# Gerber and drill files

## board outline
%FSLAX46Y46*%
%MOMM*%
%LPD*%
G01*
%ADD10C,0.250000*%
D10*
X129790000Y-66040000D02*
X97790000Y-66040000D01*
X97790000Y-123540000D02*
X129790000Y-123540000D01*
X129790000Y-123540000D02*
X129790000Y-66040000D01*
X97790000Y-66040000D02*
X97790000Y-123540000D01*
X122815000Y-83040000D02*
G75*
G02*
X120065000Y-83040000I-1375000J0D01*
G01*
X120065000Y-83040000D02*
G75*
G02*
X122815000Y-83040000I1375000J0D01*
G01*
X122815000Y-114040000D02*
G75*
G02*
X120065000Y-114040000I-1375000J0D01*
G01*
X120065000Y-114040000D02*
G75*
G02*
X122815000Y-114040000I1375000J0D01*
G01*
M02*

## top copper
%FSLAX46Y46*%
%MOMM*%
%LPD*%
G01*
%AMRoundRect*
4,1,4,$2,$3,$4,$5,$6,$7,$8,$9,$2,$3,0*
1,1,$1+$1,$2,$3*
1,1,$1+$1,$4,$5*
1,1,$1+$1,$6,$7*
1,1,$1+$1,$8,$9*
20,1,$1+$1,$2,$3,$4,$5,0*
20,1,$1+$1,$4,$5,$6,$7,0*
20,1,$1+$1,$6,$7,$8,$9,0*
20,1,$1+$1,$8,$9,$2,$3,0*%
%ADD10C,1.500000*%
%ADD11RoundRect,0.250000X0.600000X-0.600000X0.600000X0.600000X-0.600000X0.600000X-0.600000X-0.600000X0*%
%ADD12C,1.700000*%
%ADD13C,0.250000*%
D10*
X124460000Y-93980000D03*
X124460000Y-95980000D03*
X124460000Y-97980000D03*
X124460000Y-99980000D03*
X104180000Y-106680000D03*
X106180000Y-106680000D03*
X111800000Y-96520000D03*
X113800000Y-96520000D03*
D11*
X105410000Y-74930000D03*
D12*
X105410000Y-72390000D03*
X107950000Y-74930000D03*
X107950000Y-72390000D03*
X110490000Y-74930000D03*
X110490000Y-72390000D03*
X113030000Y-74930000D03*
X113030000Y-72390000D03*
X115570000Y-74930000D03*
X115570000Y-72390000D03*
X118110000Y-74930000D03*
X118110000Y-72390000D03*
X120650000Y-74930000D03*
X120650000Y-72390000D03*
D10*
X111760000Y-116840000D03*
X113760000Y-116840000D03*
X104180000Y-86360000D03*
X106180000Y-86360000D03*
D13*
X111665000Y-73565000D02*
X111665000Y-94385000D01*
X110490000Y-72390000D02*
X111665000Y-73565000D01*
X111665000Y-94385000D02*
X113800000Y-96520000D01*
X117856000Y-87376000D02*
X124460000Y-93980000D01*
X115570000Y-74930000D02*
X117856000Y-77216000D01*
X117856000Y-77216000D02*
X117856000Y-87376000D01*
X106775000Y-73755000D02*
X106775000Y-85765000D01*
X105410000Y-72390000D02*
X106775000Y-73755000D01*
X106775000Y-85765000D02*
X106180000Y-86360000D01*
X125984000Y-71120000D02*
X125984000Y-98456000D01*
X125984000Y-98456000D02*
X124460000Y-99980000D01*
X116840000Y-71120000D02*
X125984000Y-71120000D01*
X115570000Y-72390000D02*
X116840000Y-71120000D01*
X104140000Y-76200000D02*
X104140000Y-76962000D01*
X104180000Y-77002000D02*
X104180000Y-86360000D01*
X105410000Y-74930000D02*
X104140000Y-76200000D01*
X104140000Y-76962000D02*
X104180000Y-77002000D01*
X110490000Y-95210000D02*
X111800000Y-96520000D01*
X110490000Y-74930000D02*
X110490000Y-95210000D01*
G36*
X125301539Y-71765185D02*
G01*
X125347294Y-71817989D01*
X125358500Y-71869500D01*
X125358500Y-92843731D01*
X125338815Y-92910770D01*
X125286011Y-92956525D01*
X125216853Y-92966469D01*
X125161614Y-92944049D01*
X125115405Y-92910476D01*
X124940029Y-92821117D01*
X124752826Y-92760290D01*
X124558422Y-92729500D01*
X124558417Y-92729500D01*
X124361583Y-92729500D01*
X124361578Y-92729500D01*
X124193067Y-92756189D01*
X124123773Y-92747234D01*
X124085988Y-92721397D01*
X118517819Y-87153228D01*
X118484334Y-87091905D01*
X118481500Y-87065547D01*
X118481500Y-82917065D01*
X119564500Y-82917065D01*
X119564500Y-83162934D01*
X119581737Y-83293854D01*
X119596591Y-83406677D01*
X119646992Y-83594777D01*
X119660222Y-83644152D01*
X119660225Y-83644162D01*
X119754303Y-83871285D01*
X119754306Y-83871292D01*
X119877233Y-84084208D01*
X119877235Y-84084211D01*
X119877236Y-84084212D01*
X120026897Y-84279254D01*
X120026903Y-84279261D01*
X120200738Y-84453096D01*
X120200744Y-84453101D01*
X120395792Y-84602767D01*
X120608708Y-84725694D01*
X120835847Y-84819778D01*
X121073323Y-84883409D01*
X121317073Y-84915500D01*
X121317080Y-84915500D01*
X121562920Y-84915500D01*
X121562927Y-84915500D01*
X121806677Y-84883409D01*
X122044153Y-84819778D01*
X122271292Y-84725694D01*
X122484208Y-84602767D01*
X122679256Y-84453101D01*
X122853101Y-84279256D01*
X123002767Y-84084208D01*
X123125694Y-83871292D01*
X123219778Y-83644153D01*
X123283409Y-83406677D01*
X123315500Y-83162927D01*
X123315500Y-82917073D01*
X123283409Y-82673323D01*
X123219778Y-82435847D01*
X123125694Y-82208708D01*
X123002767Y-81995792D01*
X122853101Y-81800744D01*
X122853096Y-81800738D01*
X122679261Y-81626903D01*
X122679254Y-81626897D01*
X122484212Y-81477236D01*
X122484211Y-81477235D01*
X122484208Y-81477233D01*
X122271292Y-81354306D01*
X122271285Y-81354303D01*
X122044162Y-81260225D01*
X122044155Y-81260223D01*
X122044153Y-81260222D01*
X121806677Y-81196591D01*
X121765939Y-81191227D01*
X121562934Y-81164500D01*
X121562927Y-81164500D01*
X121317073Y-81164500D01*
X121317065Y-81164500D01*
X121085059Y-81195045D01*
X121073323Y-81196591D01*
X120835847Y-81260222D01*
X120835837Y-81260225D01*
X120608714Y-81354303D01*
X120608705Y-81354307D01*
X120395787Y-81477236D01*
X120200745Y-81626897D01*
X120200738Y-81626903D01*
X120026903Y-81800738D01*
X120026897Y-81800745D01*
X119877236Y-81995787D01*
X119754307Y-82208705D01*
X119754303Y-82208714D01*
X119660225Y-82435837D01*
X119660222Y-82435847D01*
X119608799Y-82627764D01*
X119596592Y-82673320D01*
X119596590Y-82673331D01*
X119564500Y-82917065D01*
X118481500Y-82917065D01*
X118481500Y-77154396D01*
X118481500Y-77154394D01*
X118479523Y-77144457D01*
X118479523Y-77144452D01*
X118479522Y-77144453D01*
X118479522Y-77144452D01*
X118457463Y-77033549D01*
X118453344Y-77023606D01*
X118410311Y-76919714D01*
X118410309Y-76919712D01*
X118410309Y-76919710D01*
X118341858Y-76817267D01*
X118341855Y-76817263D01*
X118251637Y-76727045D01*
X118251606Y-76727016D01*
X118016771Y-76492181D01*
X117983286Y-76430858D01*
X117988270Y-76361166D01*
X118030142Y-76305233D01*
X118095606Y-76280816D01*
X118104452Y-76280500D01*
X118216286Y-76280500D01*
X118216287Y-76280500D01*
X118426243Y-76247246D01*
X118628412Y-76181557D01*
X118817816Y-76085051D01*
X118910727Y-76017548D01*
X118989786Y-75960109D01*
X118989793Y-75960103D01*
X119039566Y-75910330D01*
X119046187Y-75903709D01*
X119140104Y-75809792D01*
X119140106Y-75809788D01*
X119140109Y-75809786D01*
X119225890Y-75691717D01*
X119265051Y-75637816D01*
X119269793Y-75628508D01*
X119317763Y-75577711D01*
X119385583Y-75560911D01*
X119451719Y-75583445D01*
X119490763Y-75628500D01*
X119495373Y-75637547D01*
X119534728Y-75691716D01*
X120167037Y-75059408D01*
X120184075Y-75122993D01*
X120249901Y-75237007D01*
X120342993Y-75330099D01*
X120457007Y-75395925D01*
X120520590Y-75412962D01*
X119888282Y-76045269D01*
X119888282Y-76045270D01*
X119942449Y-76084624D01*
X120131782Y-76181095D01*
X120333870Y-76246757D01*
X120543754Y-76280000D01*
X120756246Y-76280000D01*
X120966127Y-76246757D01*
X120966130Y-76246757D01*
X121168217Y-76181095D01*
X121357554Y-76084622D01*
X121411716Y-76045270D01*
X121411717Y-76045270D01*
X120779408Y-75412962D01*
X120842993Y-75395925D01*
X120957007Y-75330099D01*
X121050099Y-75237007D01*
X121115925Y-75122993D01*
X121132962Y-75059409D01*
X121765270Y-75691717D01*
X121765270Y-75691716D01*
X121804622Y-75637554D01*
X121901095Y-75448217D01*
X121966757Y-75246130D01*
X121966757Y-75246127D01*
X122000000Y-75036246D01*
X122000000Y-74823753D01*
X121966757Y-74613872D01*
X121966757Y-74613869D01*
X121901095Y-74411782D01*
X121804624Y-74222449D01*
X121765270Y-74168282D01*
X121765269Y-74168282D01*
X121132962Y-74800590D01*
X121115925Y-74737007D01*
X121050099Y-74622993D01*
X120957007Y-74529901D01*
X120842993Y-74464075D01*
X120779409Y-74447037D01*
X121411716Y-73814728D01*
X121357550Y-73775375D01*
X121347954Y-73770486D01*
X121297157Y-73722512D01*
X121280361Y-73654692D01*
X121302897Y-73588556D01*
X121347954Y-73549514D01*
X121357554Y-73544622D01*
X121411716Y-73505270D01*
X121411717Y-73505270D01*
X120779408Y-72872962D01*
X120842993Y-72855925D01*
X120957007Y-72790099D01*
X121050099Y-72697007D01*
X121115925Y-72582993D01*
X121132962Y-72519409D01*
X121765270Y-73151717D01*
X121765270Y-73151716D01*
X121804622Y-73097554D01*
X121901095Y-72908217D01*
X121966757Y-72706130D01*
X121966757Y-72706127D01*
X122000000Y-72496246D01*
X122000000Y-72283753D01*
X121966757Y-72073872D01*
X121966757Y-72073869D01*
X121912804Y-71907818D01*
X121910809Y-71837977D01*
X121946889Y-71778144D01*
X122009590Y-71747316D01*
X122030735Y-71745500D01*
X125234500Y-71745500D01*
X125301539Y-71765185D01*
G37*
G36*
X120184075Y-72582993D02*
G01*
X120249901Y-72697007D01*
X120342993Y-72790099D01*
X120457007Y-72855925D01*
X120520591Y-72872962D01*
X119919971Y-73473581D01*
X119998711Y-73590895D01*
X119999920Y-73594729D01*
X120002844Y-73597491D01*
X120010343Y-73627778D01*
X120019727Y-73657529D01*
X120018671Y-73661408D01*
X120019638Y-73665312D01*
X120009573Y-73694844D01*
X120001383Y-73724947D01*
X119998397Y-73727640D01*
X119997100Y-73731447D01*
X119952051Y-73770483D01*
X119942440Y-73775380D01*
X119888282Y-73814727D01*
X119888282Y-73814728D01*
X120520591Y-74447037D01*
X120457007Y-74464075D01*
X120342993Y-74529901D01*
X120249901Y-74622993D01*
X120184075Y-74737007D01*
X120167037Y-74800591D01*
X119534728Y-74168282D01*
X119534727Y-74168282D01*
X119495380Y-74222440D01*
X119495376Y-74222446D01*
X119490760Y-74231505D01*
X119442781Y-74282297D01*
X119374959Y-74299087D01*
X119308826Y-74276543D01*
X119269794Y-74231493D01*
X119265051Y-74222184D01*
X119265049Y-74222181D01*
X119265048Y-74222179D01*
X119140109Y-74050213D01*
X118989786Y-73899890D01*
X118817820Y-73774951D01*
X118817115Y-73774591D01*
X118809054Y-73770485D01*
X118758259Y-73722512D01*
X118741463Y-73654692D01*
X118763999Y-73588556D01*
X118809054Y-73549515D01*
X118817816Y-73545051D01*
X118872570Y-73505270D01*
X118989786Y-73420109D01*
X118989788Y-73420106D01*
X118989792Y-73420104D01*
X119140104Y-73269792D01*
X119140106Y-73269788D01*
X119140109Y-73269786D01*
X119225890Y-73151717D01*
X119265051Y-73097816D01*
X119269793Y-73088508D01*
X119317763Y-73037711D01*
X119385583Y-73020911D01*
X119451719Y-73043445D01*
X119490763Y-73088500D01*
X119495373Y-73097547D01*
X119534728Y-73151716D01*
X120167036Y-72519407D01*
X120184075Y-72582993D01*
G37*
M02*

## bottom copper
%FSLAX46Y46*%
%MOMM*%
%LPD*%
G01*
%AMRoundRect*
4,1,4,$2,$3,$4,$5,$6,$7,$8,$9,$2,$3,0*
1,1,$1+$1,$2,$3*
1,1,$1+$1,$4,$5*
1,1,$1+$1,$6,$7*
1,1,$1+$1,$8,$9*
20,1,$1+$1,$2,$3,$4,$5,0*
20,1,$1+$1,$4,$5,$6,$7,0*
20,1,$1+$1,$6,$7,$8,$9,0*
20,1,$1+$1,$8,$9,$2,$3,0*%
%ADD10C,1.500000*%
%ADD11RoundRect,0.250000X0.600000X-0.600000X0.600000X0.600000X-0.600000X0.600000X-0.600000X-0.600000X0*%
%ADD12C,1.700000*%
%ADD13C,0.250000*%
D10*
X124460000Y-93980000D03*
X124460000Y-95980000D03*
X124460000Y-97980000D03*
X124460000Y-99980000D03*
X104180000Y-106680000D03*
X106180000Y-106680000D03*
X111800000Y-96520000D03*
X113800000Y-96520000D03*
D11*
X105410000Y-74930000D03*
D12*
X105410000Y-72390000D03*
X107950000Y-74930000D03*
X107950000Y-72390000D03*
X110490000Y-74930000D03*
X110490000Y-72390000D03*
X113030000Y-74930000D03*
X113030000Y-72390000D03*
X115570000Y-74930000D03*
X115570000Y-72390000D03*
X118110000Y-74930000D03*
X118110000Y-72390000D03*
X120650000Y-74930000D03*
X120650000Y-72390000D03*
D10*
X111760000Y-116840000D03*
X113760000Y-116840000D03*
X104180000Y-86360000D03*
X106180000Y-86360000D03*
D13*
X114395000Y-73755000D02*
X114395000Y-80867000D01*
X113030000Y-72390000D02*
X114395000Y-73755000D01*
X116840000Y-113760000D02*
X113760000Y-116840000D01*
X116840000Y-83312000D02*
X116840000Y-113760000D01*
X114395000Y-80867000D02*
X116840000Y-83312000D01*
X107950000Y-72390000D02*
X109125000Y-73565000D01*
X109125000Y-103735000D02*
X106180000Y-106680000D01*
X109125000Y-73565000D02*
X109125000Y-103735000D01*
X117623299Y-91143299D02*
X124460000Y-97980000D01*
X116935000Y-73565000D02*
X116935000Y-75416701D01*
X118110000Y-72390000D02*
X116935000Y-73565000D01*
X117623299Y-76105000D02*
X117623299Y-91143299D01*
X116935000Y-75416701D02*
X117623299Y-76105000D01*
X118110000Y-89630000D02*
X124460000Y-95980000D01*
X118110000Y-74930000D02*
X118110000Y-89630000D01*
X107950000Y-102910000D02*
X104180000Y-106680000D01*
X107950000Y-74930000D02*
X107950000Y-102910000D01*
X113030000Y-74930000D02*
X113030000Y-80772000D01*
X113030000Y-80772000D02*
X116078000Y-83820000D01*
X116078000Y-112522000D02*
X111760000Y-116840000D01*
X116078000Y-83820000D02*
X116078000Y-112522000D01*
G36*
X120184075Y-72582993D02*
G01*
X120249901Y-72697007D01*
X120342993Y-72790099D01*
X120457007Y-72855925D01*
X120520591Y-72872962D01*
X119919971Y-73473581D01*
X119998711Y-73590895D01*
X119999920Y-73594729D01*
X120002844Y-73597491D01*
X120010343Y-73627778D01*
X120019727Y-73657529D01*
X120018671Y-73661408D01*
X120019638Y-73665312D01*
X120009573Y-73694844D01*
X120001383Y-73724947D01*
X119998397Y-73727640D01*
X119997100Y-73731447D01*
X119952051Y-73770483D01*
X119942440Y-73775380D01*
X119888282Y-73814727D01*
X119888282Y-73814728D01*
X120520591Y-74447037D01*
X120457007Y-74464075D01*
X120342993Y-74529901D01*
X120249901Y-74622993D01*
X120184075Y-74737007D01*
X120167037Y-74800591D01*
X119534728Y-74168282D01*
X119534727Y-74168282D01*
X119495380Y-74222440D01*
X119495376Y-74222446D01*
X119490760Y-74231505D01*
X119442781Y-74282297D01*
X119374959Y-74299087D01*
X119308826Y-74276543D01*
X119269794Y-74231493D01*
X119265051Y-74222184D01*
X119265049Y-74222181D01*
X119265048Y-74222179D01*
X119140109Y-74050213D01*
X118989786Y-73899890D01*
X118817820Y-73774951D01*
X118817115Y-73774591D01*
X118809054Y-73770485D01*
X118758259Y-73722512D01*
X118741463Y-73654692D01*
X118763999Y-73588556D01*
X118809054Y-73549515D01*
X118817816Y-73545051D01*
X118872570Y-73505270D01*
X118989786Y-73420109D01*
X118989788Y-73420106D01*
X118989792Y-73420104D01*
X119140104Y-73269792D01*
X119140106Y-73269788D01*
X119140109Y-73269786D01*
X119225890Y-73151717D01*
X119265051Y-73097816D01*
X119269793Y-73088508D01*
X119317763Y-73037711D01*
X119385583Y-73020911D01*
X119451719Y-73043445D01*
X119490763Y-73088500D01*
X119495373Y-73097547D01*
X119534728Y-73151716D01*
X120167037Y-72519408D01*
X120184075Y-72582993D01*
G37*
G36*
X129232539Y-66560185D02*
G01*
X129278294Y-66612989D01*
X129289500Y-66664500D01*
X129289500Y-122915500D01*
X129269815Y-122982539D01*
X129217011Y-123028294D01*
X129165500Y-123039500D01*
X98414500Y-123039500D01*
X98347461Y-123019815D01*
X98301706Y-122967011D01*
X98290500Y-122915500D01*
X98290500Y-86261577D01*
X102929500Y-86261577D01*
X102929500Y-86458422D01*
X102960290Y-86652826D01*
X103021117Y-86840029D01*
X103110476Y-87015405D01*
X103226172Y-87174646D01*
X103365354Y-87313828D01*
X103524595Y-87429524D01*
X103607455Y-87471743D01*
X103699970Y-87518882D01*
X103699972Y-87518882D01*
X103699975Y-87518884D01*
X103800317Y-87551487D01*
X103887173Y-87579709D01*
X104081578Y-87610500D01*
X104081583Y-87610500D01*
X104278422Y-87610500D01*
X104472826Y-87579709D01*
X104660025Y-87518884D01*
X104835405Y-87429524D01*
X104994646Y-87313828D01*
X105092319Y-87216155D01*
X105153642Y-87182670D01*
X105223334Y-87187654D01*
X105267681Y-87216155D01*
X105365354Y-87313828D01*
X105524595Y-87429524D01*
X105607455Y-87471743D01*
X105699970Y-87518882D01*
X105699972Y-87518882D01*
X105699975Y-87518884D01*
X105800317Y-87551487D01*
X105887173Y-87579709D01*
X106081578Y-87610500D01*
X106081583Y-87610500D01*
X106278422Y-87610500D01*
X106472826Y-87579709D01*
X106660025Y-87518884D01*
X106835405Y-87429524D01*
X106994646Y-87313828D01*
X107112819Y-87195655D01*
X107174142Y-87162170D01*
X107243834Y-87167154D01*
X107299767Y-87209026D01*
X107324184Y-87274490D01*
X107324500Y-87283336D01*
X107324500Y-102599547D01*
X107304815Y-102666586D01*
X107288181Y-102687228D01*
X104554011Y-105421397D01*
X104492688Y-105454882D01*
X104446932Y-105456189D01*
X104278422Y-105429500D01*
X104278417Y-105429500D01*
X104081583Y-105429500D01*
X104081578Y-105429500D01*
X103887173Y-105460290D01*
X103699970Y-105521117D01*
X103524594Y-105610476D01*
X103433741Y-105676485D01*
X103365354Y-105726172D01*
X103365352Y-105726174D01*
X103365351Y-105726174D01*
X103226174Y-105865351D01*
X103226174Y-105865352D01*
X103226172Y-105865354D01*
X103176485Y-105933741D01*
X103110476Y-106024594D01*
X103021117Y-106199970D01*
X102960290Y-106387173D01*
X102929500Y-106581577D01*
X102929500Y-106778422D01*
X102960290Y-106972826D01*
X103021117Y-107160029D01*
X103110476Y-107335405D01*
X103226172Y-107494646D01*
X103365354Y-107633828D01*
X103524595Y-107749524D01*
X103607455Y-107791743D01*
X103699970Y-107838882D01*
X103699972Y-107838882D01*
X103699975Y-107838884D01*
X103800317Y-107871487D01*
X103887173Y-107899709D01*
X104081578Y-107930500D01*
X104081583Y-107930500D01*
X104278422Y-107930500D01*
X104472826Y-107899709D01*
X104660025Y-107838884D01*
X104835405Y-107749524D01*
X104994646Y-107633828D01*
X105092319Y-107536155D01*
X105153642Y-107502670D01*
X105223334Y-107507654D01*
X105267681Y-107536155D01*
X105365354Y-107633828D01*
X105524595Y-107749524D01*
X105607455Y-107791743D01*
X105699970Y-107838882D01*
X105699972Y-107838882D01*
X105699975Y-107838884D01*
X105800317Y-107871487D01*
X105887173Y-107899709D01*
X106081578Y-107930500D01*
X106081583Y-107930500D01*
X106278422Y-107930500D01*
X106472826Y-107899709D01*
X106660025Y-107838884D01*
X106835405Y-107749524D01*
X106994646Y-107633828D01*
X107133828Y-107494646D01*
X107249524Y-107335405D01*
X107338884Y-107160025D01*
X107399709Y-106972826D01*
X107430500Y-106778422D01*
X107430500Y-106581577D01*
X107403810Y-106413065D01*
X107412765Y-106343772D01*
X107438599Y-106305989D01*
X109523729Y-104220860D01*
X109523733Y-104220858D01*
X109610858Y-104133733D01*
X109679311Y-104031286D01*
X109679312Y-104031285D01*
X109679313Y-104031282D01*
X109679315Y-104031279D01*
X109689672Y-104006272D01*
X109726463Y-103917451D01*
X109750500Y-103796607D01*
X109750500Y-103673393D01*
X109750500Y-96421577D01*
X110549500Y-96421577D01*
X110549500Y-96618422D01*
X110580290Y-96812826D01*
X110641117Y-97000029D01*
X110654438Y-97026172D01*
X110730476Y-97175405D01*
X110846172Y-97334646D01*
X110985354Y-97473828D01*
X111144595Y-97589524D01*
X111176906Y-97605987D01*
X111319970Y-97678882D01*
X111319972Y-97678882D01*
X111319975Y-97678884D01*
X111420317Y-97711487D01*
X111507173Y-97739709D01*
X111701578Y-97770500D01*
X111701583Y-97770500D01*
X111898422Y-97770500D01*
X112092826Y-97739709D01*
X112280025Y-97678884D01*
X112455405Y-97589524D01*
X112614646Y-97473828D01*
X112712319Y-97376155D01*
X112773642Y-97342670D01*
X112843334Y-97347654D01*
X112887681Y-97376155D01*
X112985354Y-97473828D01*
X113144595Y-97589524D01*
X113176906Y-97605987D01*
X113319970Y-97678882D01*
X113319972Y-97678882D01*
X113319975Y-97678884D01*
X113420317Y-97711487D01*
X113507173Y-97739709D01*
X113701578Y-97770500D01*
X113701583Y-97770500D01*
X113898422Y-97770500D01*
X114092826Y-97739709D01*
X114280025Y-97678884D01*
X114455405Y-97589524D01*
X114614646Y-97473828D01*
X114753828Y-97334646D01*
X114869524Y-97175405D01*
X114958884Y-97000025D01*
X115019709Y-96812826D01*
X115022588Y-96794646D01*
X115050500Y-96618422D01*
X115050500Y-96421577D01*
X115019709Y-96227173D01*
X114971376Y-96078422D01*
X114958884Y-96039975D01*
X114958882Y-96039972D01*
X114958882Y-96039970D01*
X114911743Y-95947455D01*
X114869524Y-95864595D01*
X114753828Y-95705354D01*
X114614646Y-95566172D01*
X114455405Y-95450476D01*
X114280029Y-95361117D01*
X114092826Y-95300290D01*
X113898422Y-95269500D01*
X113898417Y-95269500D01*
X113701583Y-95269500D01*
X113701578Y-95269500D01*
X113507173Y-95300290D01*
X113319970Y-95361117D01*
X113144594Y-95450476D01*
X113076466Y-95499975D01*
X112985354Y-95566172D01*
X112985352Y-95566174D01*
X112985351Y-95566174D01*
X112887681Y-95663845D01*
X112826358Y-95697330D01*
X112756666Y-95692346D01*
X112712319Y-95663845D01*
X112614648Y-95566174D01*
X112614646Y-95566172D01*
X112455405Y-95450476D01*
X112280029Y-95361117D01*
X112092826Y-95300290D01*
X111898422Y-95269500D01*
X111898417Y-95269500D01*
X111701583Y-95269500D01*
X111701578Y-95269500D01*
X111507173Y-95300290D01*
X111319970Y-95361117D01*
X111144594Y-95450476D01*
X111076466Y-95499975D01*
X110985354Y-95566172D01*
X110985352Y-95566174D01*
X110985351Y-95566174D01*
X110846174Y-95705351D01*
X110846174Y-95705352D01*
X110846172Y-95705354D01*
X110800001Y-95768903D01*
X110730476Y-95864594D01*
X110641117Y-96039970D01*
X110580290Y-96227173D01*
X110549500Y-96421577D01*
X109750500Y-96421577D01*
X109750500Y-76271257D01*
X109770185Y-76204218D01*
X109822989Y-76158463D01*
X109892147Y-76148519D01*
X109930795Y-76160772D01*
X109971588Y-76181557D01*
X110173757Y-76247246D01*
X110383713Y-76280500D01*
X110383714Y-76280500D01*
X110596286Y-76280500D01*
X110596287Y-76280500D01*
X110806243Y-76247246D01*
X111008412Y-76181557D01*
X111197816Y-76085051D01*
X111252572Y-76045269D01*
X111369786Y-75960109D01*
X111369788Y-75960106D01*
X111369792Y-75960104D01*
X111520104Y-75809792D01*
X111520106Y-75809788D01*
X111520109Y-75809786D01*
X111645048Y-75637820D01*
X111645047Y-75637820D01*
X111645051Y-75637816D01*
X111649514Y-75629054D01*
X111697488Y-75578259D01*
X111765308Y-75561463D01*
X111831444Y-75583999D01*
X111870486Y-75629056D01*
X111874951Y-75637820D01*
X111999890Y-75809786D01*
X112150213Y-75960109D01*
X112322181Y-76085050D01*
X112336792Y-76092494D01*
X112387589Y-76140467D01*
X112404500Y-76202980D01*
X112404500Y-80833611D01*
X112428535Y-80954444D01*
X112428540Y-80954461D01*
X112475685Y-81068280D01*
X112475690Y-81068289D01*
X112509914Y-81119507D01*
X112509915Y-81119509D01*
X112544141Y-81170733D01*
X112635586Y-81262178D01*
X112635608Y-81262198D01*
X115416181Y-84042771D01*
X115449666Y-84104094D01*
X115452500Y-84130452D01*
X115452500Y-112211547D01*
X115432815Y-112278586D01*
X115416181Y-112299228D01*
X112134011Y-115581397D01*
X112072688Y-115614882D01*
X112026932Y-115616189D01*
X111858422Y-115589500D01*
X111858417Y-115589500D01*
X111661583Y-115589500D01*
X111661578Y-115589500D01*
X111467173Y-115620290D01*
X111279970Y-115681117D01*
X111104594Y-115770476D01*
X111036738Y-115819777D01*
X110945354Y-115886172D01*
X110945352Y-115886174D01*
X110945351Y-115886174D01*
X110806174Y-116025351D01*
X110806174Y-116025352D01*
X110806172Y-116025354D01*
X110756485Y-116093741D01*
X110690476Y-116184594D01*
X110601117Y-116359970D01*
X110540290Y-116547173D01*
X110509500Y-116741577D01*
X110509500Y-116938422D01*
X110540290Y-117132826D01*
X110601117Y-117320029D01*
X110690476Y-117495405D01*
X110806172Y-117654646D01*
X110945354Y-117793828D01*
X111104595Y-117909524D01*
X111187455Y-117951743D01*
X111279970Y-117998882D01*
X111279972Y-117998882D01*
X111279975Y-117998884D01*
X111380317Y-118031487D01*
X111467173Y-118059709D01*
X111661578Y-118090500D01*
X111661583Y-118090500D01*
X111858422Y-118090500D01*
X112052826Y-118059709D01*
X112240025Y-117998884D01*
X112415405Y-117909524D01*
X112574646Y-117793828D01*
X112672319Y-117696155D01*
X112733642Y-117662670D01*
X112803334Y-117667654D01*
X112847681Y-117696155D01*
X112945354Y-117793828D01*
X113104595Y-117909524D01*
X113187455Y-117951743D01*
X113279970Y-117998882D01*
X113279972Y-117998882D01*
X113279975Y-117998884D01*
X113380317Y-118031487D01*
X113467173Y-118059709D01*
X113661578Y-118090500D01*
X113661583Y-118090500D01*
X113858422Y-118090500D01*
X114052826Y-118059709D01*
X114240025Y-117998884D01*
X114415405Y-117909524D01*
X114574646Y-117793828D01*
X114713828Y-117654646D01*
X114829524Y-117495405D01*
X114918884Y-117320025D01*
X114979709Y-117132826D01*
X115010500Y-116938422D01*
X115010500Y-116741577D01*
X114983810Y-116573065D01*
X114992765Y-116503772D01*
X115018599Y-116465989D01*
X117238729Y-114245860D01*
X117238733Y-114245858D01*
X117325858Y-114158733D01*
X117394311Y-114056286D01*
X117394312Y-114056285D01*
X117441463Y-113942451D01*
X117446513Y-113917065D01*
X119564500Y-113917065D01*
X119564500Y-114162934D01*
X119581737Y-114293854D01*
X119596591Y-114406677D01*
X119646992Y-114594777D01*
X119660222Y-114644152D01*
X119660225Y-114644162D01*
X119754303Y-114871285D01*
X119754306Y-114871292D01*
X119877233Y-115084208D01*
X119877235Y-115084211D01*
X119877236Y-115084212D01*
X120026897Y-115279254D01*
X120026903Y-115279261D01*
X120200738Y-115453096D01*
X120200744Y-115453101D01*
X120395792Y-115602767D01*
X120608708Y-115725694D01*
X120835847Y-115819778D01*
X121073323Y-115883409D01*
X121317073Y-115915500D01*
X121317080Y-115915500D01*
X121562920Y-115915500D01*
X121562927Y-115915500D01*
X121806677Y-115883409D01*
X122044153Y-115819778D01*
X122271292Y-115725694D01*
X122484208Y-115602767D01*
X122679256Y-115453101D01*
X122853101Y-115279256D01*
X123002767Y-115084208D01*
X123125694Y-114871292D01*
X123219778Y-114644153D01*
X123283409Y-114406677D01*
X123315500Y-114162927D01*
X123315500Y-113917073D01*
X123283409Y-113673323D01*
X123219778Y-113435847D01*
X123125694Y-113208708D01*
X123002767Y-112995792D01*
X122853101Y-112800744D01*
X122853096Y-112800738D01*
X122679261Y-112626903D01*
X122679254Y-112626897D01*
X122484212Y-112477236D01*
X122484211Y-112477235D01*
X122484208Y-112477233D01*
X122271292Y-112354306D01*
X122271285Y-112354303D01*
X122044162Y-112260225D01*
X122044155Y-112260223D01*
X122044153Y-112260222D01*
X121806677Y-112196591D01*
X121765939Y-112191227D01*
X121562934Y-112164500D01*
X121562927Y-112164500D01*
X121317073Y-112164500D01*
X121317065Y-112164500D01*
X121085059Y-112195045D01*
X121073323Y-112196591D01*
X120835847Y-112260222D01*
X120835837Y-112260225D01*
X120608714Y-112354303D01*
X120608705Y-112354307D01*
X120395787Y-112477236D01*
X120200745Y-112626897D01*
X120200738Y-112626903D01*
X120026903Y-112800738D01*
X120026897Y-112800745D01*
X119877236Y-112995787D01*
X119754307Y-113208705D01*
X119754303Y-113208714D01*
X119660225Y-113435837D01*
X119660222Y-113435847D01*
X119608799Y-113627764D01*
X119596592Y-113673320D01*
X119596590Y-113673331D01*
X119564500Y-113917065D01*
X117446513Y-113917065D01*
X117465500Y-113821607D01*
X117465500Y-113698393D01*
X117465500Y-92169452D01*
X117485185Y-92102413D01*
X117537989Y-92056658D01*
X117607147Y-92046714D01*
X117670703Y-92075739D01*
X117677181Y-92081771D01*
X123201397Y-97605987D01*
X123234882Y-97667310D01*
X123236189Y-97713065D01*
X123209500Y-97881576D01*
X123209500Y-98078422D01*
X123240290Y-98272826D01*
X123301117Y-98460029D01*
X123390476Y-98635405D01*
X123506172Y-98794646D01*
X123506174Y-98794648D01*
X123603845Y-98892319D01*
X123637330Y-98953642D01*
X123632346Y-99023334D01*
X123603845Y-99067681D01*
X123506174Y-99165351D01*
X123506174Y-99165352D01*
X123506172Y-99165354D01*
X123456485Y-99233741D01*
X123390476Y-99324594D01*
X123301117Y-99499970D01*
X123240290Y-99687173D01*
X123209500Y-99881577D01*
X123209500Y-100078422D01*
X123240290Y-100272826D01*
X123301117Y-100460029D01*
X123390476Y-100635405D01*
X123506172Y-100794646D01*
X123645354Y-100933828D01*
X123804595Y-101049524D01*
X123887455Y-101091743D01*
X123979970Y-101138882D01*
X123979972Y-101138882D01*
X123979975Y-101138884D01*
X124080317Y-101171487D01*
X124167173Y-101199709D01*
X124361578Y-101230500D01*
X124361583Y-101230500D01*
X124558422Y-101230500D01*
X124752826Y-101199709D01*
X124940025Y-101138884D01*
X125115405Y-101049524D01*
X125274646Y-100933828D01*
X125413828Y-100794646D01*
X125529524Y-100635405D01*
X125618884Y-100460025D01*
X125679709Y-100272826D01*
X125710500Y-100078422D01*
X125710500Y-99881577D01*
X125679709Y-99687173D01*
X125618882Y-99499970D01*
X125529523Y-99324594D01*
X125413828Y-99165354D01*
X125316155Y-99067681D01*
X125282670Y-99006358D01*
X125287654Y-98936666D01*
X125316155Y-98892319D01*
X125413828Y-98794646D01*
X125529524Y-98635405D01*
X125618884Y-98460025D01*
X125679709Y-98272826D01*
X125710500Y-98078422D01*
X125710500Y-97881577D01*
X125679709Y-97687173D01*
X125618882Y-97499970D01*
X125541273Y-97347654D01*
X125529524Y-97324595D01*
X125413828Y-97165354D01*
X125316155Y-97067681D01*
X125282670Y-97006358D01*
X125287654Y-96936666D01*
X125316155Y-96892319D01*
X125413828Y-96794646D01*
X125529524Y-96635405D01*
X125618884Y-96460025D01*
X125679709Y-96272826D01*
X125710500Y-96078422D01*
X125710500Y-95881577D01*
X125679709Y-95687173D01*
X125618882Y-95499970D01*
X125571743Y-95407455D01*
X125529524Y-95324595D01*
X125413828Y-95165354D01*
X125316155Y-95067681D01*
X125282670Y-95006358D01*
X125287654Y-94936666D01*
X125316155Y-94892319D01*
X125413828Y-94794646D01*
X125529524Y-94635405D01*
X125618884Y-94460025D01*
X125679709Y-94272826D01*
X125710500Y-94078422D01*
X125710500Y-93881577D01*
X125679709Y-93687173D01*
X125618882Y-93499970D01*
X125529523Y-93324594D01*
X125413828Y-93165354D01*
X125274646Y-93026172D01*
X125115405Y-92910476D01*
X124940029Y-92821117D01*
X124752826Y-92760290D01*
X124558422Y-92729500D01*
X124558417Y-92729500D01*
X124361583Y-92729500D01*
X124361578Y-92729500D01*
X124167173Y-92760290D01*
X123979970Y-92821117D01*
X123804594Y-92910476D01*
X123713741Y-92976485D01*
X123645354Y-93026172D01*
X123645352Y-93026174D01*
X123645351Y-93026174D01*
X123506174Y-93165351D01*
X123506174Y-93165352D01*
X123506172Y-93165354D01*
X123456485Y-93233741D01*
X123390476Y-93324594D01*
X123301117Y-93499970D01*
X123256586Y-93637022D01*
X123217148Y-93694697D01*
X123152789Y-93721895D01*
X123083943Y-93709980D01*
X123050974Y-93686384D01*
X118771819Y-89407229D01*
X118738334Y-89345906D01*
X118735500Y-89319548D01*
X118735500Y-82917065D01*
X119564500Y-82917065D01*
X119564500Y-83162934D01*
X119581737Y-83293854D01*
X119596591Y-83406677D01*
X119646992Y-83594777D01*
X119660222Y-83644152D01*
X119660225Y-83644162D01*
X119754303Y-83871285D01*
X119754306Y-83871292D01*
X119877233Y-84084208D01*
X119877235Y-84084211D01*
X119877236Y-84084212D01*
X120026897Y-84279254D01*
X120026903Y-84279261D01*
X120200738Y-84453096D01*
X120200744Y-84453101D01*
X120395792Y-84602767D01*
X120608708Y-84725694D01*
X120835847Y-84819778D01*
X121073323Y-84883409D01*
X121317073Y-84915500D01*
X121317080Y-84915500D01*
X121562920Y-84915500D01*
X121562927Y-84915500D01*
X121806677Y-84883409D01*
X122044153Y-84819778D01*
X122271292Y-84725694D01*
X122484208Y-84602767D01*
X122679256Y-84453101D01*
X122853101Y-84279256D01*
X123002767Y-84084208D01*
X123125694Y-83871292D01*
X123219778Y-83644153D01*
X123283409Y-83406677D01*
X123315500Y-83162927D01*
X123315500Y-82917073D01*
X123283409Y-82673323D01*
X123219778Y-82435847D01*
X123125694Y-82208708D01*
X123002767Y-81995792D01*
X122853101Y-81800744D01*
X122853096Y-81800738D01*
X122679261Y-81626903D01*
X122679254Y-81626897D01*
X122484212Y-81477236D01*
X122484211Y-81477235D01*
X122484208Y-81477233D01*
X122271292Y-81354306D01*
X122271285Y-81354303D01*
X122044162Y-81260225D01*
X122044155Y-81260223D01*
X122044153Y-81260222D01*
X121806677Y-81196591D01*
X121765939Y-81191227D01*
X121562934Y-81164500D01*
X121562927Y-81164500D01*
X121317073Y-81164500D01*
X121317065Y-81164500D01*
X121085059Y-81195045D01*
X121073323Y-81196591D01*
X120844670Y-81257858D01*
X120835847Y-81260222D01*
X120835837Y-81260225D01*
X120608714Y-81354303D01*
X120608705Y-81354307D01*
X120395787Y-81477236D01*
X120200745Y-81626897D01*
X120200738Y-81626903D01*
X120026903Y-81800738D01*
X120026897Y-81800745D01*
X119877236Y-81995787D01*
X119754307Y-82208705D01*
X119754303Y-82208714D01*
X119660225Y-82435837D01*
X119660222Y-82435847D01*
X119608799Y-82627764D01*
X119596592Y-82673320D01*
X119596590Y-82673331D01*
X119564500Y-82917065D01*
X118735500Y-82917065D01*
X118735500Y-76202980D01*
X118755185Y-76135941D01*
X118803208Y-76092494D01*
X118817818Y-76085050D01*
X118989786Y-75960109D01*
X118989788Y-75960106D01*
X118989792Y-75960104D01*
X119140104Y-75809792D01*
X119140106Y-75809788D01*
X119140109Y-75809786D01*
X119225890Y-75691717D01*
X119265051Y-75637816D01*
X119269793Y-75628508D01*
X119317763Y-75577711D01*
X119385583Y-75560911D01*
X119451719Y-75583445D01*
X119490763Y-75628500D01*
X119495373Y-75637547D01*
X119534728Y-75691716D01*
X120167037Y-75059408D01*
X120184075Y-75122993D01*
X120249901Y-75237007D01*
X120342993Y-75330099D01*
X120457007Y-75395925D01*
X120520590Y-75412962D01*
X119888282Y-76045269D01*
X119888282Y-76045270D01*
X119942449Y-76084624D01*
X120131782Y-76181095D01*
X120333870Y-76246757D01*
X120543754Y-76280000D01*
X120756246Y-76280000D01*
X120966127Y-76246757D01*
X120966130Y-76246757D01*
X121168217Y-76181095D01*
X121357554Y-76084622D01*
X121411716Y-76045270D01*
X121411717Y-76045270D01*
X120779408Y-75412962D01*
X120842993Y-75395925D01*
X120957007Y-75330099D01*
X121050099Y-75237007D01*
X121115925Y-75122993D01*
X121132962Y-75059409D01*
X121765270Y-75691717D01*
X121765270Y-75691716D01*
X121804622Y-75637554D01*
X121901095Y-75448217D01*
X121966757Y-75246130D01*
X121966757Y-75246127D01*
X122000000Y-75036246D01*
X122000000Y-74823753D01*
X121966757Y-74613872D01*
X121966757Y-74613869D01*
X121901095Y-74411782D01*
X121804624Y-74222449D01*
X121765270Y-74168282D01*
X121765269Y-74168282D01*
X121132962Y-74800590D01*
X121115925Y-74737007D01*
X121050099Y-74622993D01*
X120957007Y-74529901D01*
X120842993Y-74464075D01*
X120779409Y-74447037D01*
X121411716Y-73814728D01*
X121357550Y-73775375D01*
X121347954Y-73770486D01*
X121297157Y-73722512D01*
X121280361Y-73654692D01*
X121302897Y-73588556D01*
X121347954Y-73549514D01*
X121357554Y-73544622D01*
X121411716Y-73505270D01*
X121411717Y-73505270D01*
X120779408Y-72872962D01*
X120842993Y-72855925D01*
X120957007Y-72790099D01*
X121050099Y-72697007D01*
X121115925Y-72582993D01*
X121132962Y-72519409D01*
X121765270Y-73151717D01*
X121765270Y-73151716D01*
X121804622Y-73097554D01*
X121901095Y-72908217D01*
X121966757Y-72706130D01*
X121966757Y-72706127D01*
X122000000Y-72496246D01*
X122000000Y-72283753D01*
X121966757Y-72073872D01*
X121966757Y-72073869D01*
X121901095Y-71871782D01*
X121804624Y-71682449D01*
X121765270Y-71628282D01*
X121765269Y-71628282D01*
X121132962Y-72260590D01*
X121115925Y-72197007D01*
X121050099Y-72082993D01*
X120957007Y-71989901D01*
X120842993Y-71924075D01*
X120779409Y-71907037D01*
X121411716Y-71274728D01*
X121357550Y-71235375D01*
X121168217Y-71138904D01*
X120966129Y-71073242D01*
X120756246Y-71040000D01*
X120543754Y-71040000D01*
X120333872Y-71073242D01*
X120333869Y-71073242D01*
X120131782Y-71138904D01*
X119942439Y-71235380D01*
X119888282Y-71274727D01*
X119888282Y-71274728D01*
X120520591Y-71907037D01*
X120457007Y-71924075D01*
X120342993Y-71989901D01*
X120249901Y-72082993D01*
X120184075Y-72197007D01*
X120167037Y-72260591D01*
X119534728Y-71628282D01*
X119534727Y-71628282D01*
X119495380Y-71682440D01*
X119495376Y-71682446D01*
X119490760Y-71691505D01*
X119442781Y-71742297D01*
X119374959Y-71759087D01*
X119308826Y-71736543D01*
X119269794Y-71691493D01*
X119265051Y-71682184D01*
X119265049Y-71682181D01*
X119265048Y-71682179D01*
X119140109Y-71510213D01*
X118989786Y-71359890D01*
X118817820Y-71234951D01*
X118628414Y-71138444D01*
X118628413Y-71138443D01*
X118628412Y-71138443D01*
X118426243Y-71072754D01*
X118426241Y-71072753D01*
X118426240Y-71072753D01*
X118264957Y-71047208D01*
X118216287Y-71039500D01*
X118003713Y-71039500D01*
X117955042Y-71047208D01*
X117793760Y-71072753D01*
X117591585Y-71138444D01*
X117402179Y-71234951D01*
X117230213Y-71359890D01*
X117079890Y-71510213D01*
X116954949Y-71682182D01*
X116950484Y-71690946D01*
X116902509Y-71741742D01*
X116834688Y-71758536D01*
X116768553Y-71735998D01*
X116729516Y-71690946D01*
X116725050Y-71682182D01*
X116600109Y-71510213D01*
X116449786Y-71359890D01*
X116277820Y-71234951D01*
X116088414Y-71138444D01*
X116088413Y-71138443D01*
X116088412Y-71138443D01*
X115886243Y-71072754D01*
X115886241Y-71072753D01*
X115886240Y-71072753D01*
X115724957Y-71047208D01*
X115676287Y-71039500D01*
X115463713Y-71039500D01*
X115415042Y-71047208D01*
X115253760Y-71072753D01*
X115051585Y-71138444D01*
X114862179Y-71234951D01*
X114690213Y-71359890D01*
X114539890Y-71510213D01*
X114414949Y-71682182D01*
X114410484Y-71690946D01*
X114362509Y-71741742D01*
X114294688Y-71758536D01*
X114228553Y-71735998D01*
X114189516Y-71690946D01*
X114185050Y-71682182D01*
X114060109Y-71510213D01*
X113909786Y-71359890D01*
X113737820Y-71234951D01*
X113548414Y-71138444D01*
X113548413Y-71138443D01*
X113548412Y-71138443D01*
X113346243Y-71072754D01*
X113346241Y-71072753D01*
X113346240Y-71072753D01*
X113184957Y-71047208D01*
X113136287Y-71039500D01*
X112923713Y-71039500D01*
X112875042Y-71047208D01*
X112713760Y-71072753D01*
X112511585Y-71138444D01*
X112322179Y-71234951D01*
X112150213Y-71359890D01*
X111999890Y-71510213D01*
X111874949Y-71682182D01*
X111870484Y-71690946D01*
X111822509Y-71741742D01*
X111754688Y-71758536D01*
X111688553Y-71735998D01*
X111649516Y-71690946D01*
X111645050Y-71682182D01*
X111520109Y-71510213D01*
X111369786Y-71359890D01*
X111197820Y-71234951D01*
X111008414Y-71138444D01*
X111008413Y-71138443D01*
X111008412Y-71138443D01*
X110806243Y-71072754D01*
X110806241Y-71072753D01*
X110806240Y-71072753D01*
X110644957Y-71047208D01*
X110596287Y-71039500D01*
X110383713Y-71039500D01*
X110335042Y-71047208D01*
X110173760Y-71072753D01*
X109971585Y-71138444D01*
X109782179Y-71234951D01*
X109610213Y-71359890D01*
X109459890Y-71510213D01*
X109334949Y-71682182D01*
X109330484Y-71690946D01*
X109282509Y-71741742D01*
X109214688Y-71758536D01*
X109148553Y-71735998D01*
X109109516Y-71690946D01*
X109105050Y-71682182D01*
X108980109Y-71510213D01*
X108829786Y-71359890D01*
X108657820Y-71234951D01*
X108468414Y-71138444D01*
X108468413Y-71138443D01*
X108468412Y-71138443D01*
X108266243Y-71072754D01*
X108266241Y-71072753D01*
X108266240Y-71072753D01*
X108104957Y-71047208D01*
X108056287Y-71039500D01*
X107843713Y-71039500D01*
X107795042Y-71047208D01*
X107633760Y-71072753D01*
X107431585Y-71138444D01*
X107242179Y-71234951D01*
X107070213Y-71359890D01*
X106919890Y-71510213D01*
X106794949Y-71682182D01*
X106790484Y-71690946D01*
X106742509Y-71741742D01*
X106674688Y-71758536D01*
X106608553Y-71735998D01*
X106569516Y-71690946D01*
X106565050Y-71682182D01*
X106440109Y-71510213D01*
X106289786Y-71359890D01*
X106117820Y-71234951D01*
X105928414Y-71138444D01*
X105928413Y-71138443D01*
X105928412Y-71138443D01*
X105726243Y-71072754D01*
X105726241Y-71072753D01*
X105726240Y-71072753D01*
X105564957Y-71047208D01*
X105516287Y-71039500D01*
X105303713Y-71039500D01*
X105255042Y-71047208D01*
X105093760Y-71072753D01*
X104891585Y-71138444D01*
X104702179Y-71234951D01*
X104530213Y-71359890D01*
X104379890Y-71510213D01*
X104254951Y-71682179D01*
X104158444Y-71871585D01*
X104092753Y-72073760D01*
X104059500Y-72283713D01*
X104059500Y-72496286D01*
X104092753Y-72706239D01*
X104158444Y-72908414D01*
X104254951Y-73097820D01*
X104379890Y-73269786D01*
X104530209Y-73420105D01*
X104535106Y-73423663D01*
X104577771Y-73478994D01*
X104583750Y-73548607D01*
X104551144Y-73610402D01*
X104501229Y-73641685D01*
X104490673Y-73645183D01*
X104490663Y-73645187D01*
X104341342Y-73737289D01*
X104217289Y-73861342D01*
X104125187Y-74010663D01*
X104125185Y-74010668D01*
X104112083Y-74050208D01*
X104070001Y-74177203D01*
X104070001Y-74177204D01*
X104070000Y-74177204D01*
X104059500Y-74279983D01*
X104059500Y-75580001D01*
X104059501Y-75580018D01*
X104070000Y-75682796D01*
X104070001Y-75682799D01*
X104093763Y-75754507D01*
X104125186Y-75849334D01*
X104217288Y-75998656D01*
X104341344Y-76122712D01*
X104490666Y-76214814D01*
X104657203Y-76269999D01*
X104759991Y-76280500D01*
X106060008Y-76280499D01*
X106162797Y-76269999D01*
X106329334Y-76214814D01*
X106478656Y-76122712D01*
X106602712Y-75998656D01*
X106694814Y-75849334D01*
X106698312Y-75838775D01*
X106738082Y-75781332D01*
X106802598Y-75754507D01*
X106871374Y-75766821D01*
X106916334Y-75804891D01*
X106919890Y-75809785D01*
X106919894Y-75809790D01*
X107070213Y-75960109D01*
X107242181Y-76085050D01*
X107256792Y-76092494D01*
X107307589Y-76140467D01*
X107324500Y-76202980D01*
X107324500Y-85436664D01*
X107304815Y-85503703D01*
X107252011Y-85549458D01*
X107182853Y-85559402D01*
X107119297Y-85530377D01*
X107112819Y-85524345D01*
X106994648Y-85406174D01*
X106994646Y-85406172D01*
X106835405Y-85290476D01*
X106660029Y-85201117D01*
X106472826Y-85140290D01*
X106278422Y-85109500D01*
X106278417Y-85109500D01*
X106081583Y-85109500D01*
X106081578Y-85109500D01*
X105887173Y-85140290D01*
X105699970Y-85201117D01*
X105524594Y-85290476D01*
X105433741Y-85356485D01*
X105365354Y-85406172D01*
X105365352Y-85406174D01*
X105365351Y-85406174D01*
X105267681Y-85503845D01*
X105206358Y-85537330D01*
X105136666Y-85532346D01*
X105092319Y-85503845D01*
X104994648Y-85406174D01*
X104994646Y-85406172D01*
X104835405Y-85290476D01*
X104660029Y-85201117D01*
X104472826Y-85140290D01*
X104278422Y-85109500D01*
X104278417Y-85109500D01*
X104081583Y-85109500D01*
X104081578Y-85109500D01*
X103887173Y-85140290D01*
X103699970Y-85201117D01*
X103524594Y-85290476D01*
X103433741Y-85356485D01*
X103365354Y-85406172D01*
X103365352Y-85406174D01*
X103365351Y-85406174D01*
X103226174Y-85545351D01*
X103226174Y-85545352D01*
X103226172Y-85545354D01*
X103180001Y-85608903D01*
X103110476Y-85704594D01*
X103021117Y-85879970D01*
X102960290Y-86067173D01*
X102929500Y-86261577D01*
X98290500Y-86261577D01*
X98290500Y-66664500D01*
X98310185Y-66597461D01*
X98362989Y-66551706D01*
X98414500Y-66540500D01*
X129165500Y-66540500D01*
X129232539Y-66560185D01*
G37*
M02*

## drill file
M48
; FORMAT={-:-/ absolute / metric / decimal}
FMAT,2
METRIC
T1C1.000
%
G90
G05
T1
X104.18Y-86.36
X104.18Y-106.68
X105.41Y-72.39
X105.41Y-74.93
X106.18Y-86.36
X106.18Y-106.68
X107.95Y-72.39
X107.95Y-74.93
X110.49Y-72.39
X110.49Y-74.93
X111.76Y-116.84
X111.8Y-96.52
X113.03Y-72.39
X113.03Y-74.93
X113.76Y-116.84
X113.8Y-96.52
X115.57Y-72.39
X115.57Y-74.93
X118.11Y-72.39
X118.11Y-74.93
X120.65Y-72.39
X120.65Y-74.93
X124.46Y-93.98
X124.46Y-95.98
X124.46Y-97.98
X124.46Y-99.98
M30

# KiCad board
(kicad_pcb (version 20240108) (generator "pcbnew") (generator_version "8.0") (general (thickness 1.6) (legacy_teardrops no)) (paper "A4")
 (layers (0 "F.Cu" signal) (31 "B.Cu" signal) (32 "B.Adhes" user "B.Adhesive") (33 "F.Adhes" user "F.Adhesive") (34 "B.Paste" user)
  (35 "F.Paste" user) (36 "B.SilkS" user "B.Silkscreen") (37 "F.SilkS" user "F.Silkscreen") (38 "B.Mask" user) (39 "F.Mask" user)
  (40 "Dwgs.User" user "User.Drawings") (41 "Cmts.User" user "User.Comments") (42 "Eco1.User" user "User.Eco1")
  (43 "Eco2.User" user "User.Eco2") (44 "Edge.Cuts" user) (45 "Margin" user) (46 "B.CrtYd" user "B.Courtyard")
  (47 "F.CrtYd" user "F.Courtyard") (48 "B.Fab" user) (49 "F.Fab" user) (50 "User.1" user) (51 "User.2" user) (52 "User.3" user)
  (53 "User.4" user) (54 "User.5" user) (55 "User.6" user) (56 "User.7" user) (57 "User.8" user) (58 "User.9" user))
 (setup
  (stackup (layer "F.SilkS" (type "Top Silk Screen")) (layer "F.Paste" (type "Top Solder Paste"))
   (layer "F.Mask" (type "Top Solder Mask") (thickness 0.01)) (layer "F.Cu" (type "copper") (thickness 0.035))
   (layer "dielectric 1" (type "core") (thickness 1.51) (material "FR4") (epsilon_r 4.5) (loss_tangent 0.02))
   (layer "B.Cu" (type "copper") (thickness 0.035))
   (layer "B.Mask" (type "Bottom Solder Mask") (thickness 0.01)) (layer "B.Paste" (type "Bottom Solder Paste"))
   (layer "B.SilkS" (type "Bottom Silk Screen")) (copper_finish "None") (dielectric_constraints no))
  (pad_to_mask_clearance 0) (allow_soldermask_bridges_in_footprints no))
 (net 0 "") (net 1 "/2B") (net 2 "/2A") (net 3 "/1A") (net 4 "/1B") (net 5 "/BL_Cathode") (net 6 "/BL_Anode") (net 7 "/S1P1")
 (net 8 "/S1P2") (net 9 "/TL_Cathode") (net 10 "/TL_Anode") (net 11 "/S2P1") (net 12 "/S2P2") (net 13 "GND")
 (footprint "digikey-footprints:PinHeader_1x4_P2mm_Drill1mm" (layer "F.Cu") (at 124.46 93.98 -90)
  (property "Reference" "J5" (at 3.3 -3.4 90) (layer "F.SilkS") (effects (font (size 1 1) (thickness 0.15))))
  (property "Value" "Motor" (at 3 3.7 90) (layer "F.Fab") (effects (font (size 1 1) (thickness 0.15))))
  (pad "1" thru_hole circle (at 0 0 270) (size 1.5 1.5) (drill 1) (layers "*.Cu" "*.Mask") (remove_unused_layers no) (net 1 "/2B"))
  (pad "2" thru_hole circle (at 2 0 270) (size 1.5 1.5) (drill 1) (layers "*.Cu" "*.Mask") (remove_unused_layers no) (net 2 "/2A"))
  (pad "3" thru_hole circle (at 4 0 270) (size 1.5 1.5) (drill 1) (layers "*.Cu" "*.Mask") (remove_unused_layers no) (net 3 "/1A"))
  (pad "4" thru_hole circle (at 6 0 270) (size 1.5 1.5) (drill 1) (layers "*.Cu" "*.Mask") (remove_unused_layers no) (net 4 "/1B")))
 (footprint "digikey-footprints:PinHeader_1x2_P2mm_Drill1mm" (layer "F.Cu") (at 104.18 106.68)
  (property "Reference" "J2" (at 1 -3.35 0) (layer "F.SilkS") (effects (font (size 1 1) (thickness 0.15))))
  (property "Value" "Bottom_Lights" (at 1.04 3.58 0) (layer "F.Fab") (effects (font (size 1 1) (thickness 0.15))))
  (pad "1" thru_hole circle (at 0 0) (size 1.5 1.5) (drill 1) (layers "*.Cu" "*.Mask") (remove_unused_layers no) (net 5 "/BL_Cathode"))
  (pad "2" thru_hole circle (at 2 0) (size 1.5 1.5) (drill 1) (layers "*.Cu" "*.Mask") (remove_unused_layers no) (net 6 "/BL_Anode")))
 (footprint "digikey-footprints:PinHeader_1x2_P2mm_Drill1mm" (layer "F.Cu") (at 111.8 96.52)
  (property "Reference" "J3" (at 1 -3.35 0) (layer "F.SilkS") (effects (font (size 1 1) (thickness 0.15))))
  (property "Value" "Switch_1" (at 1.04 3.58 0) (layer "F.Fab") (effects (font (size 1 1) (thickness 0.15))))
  (pad "1" thru_hole circle (at 0 0) (size 1.5 1.5) (drill 1) (layers "*.Cu" "*.Mask") (remove_unused_layers no) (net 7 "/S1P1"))
  (pad "2" thru_hole circle (at 2 0) (size 1.5 1.5) (drill 1) (layers "*.Cu" "*.Mask") (remove_unused_layers no) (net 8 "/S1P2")))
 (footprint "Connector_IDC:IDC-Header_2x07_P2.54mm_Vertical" (layer "F.Cu") (at 105.41 74.93 90)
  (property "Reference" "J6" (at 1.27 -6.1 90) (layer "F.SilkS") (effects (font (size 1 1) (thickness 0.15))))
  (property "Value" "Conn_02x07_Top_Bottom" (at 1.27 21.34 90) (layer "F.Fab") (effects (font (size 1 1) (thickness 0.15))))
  (pad "1" thru_hole roundrect (at 0 0 90) (size 1.7 1.7) (drill 1) (layers "*.Cu" "*.Mask") (remove_unused_layers no)
   (roundrect_rratio 0.147059) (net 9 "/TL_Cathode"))
  (pad "2" thru_hole circle (at 2.54 0 90) (size 1.7 1.7) (drill 1) (layers "*.Cu" "*.Mask") (remove_unused_layers no) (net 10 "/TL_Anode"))
  (pad "3" thru_hole circle (at 0 2.54 90) (size 1.7 1.7) (drill 1) (layers "*.Cu" "*.Mask") (remove_unused_layers no) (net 5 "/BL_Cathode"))
  (pad "4" thru_hole circle (at 2.54 2.54 90) (size 1.7 1.7) (drill 1) (layers "*.Cu" "*.Mask") (remove_unused_layers no)
   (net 6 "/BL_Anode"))
  (pad "5" thru_hole circle (at 0 5.08 90) (size 1.7 1.7) (drill 1) (layers "*.Cu" "*.Mask") (remove_unused_layers no) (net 7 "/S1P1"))
  (pad "6" thru_hole circle (at 2.54 5.08 90) (size 1.7 1.7) (drill 1) (layers "*.Cu" "*.Mask") (remove_unused_layers no) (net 8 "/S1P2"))
  (pad "7" thru_hole circle (at 0 7.62 90) (size 1.7 1.7) (drill 1) (layers "*.Cu" "*.Mask") (remove_unused_layers no) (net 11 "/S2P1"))
  (pad "8" thru_hole circle (at 2.54 7.62 90) (size 1.7 1.7) (drill 1) (layers "*.Cu" "*.Mask") (remove_unused_layers no) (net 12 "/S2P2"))
  (pad "9" thru_hole circle (at 0 10.16 90) (size 1.7 1.7) (drill 1) (layers "*.Cu" "*.Mask") (remove_unused_layers no) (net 1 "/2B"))
  (pad "10" thru_hole circle (at 2.54 10.16 90) (size 1.7 1.7) (drill 1) (layers "*.Cu" "*.Mask") (remove_unused_layers no) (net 4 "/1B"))
  (pad "11" thru_hole circle (at 0 12.7 90) (size 1.7 1.7) (drill 1) (layers "*.Cu" "*.Mask") (remove_unused_layers no) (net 2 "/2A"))
  (pad "12" thru_hole circle (at 2.54 12.7 90) (size 1.7 1.7) (drill 1) (layers "*.Cu" "*.Mask") (remove_unused_layers no) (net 3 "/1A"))
  (pad "13" thru_hole circle (at 0 15.24 90) (size 1.7 1.7) (drill 1) (layers "*.Cu" "*.Mask") (remove_unused_layers no) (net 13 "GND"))
  (pad "14" thru_hole circle (at 2.54 15.24 90) (size 1.7 1.7) (drill 1) (layers "*.Cu" "*.Mask") (remove_unused_layers no) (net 13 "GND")))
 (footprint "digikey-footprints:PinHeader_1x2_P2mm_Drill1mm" (layer "F.Cu") (at 111.76 116.84)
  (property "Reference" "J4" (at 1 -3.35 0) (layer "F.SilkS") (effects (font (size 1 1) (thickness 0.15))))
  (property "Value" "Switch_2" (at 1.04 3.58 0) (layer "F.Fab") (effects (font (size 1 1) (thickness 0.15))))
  (pad "1" thru_hole circle (at 0 0) (size 1.5 1.5) (drill 1) (layers "*.Cu" "*.Mask") (remove_unused_layers no) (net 11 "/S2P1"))
  (pad "2" thru_hole circle (at 2 0) (size 1.5 1.5) (drill 1) (layers "*.Cu" "*.Mask") (remove_unused_layers no) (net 12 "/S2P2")))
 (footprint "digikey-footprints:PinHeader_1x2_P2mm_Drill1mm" (layer "F.Cu") (at 104.18 86.36)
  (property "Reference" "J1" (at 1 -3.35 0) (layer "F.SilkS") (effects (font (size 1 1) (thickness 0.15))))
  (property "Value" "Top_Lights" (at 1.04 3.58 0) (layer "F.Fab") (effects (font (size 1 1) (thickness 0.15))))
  (pad "1" thru_hole circle (at 0 0) (size 1.5 1.5) (drill 1) (layers "*.Cu" "*.Mask") (remove_unused_layers no) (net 9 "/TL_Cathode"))
  (pad "2" thru_hole circle (at 2 0) (size 1.5 1.5) (drill 1) (layers "*.Cu" "*.Mask") (remove_unused_layers no) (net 10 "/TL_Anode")))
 (gr_line (start 129.79 66.04) (end 97.79 66.04) (stroke (width 0.25) (type default)) (layer "Edge.Cuts"))
 (gr_line (start 97.79 123.54) (end 129.79 123.54) (stroke (width 0.25) (type default)) (layer "Edge.Cuts"))
 (gr_line (start 129.79 123.54) (end 129.79 66.04) (stroke (width 0.25) (type default)) (layer "Edge.Cuts"))
 (gr_line (start 97.79 66.04) (end 97.79 123.54) (stroke (width 0.25) (type default)) (layer "Edge.Cuts"))
 (gr_circle (center 121.44 83.04) (end 122.815 83.04) (stroke (width 0.25) (type default)) (fill none) (layer "Edge.Cuts"))
 (gr_circle (center 121.44 114.04) (end 122.815 114.04) (stroke (width 0.25) (type default)) (fill none) (layer "Edge.Cuts"))
 (segment (start 111.665 73.565) (end 111.665 94.385) (width 0.25) (layer "F.Cu") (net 8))
 (segment (start 110.49 72.39) (end 111.665 73.565) (width 0.25) (layer "F.Cu") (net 8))
 (segment (start 111.665 94.385) (end 113.8 96.52) (width 0.25) (layer "F.Cu") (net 8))
 (segment (start 114.395 73.755) (end 114.395 80.867) (width 0.25) (layer "B.Cu") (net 12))
 (segment (start 113.03 72.39) (end 114.395 73.755) (width 0.25) (layer "B.Cu") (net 12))
 (segment (start 116.84 113.76) (end 113.76 116.84) (width 0.25) (layer "B.Cu") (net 12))
 (segment (start 116.84 83.312) (end 116.84 113.76) (width 0.25) (layer "B.Cu") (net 12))
 (segment (start 114.395 80.867) (end 116.84 83.312) (width 0.25) (layer "B.Cu") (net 12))
 (segment (start 107.95 72.39) (end 109.125 73.565) (width 0.25) (layer "B.Cu") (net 6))
 (segment (start 109.125 103.735) (end 106.18 106.68) (width 0.25) (layer "B.Cu") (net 6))
 (segment (start 109.125 73.565) (end 109.125 103.735) (width 0.25) (layer "B.Cu") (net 6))
 (segment (start 117.856 87.376) (end 124.46 93.98) (width 0.25) (layer "F.Cu") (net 1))
 (segment (start 115.57 74.93) (end 117.856 77.216) (width 0.25) (layer "F.Cu") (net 1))
 (segment (start 117.856 77.216) (end 117.856 87.376) (width 0.25) (layer "F.Cu") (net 1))
 (segment (start 117.623299 91.143299) (end 124.46 97.98) (width 0.25) (layer "B.Cu") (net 3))
 (segment (start 116.935 73.565) (end 116.935 75.416701) (width 0.25) (layer "B.Cu") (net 3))
 (segment (start 118.11 72.39) (end 116.935 73.565) (width 0.25) (layer "B.Cu") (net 3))
 (segment (start 117.623299 76.105) (end 117.623299 91.143299) (width 0.25) (layer "B.Cu") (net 3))
 (segment (start 116.935 75.416701) (end 117.623299 76.105) (width 0.25) (layer "B.Cu") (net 3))
 (segment (start 118.11 89.63) (end 124.46 95.98) (width 0.25) (layer "B.Cu") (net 2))
 (segment (start 118.11 74.93) (end 118.11 89.63) (width 0.25) (layer "B.Cu") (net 2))
 (segment (start 107.95 102.91) (end 104.18 106.68) (width 0.25) (layer "B.Cu") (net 5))
 (segment (start 107.95 74.93) (end 107.95 102.91) (width 0.25) (layer "B.Cu") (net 5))
 (segment (start 106.775 73.755) (end 106.775 85.765) (width 0.25) (layer "F.Cu") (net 10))
 (segment (start 105.41 72.39) (end 106.775 73.755) (width 0.25) (layer "F.Cu") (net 10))
 (segment (start 106.775 85.765) (end 106.18 86.36) (width 0.25) (layer "F.Cu") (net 10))
 (segment (start 113.03 74.93) (end 113.03 80.772) (width 0.25) (layer "B.Cu") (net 11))
 (segment (start 113.03 80.772) (end 116.078 83.82) (width 0.25) (layer "B.Cu") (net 11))
 (segment (start 116.078 112.522) (end 111.76 116.84) (width 0.25) (layer "B.Cu") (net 11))
 (segment (start 116.078 83.82) (end 116.078 112.522) (width 0.25) (layer "B.Cu") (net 11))
 (segment (start 125.984 71.12) (end 125.984 98.456) (width 0.25) (layer "F.Cu") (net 4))
 (segment (start 125.984 98.456) (end 124.46 99.98) (width 0.25) (layer "F.Cu") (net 4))
 (segment (start 116.84 71.12) (end 125.984 71.12) (width 0.25) (layer "F.Cu") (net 4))
 (segment (start 115.57 72.39) (end 116.84 71.12) (width 0.25) (layer "F.Cu") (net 4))
 (segment (start 104.14 76.2) (end 104.14 76.962) (width 0.25) (layer "F.Cu") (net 9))
 (segment (start 104.18 77.002) (end 104.18 86.36) (width 0.25) (layer "F.Cu") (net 9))
 (segment (start 105.41 74.93) (end 104.14 76.2) (width 0.25) (layer "F.Cu") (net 9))
 (segment (start 104.14 76.962) (end 104.18 77.002) (width 0.25) (layer "F.Cu") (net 9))
 (segment (start 110.49 95.21) (end 111.8 96.52) (width 0.25) (layer "F.Cu") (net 7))
 (segment (start 110.49 74.93) (end 110.49 95.21) (width 0.25) (layer "F.Cu") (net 7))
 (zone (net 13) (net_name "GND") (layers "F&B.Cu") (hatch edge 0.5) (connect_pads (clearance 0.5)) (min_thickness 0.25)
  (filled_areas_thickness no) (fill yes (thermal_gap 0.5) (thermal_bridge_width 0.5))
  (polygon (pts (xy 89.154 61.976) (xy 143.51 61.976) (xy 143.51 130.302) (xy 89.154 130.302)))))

